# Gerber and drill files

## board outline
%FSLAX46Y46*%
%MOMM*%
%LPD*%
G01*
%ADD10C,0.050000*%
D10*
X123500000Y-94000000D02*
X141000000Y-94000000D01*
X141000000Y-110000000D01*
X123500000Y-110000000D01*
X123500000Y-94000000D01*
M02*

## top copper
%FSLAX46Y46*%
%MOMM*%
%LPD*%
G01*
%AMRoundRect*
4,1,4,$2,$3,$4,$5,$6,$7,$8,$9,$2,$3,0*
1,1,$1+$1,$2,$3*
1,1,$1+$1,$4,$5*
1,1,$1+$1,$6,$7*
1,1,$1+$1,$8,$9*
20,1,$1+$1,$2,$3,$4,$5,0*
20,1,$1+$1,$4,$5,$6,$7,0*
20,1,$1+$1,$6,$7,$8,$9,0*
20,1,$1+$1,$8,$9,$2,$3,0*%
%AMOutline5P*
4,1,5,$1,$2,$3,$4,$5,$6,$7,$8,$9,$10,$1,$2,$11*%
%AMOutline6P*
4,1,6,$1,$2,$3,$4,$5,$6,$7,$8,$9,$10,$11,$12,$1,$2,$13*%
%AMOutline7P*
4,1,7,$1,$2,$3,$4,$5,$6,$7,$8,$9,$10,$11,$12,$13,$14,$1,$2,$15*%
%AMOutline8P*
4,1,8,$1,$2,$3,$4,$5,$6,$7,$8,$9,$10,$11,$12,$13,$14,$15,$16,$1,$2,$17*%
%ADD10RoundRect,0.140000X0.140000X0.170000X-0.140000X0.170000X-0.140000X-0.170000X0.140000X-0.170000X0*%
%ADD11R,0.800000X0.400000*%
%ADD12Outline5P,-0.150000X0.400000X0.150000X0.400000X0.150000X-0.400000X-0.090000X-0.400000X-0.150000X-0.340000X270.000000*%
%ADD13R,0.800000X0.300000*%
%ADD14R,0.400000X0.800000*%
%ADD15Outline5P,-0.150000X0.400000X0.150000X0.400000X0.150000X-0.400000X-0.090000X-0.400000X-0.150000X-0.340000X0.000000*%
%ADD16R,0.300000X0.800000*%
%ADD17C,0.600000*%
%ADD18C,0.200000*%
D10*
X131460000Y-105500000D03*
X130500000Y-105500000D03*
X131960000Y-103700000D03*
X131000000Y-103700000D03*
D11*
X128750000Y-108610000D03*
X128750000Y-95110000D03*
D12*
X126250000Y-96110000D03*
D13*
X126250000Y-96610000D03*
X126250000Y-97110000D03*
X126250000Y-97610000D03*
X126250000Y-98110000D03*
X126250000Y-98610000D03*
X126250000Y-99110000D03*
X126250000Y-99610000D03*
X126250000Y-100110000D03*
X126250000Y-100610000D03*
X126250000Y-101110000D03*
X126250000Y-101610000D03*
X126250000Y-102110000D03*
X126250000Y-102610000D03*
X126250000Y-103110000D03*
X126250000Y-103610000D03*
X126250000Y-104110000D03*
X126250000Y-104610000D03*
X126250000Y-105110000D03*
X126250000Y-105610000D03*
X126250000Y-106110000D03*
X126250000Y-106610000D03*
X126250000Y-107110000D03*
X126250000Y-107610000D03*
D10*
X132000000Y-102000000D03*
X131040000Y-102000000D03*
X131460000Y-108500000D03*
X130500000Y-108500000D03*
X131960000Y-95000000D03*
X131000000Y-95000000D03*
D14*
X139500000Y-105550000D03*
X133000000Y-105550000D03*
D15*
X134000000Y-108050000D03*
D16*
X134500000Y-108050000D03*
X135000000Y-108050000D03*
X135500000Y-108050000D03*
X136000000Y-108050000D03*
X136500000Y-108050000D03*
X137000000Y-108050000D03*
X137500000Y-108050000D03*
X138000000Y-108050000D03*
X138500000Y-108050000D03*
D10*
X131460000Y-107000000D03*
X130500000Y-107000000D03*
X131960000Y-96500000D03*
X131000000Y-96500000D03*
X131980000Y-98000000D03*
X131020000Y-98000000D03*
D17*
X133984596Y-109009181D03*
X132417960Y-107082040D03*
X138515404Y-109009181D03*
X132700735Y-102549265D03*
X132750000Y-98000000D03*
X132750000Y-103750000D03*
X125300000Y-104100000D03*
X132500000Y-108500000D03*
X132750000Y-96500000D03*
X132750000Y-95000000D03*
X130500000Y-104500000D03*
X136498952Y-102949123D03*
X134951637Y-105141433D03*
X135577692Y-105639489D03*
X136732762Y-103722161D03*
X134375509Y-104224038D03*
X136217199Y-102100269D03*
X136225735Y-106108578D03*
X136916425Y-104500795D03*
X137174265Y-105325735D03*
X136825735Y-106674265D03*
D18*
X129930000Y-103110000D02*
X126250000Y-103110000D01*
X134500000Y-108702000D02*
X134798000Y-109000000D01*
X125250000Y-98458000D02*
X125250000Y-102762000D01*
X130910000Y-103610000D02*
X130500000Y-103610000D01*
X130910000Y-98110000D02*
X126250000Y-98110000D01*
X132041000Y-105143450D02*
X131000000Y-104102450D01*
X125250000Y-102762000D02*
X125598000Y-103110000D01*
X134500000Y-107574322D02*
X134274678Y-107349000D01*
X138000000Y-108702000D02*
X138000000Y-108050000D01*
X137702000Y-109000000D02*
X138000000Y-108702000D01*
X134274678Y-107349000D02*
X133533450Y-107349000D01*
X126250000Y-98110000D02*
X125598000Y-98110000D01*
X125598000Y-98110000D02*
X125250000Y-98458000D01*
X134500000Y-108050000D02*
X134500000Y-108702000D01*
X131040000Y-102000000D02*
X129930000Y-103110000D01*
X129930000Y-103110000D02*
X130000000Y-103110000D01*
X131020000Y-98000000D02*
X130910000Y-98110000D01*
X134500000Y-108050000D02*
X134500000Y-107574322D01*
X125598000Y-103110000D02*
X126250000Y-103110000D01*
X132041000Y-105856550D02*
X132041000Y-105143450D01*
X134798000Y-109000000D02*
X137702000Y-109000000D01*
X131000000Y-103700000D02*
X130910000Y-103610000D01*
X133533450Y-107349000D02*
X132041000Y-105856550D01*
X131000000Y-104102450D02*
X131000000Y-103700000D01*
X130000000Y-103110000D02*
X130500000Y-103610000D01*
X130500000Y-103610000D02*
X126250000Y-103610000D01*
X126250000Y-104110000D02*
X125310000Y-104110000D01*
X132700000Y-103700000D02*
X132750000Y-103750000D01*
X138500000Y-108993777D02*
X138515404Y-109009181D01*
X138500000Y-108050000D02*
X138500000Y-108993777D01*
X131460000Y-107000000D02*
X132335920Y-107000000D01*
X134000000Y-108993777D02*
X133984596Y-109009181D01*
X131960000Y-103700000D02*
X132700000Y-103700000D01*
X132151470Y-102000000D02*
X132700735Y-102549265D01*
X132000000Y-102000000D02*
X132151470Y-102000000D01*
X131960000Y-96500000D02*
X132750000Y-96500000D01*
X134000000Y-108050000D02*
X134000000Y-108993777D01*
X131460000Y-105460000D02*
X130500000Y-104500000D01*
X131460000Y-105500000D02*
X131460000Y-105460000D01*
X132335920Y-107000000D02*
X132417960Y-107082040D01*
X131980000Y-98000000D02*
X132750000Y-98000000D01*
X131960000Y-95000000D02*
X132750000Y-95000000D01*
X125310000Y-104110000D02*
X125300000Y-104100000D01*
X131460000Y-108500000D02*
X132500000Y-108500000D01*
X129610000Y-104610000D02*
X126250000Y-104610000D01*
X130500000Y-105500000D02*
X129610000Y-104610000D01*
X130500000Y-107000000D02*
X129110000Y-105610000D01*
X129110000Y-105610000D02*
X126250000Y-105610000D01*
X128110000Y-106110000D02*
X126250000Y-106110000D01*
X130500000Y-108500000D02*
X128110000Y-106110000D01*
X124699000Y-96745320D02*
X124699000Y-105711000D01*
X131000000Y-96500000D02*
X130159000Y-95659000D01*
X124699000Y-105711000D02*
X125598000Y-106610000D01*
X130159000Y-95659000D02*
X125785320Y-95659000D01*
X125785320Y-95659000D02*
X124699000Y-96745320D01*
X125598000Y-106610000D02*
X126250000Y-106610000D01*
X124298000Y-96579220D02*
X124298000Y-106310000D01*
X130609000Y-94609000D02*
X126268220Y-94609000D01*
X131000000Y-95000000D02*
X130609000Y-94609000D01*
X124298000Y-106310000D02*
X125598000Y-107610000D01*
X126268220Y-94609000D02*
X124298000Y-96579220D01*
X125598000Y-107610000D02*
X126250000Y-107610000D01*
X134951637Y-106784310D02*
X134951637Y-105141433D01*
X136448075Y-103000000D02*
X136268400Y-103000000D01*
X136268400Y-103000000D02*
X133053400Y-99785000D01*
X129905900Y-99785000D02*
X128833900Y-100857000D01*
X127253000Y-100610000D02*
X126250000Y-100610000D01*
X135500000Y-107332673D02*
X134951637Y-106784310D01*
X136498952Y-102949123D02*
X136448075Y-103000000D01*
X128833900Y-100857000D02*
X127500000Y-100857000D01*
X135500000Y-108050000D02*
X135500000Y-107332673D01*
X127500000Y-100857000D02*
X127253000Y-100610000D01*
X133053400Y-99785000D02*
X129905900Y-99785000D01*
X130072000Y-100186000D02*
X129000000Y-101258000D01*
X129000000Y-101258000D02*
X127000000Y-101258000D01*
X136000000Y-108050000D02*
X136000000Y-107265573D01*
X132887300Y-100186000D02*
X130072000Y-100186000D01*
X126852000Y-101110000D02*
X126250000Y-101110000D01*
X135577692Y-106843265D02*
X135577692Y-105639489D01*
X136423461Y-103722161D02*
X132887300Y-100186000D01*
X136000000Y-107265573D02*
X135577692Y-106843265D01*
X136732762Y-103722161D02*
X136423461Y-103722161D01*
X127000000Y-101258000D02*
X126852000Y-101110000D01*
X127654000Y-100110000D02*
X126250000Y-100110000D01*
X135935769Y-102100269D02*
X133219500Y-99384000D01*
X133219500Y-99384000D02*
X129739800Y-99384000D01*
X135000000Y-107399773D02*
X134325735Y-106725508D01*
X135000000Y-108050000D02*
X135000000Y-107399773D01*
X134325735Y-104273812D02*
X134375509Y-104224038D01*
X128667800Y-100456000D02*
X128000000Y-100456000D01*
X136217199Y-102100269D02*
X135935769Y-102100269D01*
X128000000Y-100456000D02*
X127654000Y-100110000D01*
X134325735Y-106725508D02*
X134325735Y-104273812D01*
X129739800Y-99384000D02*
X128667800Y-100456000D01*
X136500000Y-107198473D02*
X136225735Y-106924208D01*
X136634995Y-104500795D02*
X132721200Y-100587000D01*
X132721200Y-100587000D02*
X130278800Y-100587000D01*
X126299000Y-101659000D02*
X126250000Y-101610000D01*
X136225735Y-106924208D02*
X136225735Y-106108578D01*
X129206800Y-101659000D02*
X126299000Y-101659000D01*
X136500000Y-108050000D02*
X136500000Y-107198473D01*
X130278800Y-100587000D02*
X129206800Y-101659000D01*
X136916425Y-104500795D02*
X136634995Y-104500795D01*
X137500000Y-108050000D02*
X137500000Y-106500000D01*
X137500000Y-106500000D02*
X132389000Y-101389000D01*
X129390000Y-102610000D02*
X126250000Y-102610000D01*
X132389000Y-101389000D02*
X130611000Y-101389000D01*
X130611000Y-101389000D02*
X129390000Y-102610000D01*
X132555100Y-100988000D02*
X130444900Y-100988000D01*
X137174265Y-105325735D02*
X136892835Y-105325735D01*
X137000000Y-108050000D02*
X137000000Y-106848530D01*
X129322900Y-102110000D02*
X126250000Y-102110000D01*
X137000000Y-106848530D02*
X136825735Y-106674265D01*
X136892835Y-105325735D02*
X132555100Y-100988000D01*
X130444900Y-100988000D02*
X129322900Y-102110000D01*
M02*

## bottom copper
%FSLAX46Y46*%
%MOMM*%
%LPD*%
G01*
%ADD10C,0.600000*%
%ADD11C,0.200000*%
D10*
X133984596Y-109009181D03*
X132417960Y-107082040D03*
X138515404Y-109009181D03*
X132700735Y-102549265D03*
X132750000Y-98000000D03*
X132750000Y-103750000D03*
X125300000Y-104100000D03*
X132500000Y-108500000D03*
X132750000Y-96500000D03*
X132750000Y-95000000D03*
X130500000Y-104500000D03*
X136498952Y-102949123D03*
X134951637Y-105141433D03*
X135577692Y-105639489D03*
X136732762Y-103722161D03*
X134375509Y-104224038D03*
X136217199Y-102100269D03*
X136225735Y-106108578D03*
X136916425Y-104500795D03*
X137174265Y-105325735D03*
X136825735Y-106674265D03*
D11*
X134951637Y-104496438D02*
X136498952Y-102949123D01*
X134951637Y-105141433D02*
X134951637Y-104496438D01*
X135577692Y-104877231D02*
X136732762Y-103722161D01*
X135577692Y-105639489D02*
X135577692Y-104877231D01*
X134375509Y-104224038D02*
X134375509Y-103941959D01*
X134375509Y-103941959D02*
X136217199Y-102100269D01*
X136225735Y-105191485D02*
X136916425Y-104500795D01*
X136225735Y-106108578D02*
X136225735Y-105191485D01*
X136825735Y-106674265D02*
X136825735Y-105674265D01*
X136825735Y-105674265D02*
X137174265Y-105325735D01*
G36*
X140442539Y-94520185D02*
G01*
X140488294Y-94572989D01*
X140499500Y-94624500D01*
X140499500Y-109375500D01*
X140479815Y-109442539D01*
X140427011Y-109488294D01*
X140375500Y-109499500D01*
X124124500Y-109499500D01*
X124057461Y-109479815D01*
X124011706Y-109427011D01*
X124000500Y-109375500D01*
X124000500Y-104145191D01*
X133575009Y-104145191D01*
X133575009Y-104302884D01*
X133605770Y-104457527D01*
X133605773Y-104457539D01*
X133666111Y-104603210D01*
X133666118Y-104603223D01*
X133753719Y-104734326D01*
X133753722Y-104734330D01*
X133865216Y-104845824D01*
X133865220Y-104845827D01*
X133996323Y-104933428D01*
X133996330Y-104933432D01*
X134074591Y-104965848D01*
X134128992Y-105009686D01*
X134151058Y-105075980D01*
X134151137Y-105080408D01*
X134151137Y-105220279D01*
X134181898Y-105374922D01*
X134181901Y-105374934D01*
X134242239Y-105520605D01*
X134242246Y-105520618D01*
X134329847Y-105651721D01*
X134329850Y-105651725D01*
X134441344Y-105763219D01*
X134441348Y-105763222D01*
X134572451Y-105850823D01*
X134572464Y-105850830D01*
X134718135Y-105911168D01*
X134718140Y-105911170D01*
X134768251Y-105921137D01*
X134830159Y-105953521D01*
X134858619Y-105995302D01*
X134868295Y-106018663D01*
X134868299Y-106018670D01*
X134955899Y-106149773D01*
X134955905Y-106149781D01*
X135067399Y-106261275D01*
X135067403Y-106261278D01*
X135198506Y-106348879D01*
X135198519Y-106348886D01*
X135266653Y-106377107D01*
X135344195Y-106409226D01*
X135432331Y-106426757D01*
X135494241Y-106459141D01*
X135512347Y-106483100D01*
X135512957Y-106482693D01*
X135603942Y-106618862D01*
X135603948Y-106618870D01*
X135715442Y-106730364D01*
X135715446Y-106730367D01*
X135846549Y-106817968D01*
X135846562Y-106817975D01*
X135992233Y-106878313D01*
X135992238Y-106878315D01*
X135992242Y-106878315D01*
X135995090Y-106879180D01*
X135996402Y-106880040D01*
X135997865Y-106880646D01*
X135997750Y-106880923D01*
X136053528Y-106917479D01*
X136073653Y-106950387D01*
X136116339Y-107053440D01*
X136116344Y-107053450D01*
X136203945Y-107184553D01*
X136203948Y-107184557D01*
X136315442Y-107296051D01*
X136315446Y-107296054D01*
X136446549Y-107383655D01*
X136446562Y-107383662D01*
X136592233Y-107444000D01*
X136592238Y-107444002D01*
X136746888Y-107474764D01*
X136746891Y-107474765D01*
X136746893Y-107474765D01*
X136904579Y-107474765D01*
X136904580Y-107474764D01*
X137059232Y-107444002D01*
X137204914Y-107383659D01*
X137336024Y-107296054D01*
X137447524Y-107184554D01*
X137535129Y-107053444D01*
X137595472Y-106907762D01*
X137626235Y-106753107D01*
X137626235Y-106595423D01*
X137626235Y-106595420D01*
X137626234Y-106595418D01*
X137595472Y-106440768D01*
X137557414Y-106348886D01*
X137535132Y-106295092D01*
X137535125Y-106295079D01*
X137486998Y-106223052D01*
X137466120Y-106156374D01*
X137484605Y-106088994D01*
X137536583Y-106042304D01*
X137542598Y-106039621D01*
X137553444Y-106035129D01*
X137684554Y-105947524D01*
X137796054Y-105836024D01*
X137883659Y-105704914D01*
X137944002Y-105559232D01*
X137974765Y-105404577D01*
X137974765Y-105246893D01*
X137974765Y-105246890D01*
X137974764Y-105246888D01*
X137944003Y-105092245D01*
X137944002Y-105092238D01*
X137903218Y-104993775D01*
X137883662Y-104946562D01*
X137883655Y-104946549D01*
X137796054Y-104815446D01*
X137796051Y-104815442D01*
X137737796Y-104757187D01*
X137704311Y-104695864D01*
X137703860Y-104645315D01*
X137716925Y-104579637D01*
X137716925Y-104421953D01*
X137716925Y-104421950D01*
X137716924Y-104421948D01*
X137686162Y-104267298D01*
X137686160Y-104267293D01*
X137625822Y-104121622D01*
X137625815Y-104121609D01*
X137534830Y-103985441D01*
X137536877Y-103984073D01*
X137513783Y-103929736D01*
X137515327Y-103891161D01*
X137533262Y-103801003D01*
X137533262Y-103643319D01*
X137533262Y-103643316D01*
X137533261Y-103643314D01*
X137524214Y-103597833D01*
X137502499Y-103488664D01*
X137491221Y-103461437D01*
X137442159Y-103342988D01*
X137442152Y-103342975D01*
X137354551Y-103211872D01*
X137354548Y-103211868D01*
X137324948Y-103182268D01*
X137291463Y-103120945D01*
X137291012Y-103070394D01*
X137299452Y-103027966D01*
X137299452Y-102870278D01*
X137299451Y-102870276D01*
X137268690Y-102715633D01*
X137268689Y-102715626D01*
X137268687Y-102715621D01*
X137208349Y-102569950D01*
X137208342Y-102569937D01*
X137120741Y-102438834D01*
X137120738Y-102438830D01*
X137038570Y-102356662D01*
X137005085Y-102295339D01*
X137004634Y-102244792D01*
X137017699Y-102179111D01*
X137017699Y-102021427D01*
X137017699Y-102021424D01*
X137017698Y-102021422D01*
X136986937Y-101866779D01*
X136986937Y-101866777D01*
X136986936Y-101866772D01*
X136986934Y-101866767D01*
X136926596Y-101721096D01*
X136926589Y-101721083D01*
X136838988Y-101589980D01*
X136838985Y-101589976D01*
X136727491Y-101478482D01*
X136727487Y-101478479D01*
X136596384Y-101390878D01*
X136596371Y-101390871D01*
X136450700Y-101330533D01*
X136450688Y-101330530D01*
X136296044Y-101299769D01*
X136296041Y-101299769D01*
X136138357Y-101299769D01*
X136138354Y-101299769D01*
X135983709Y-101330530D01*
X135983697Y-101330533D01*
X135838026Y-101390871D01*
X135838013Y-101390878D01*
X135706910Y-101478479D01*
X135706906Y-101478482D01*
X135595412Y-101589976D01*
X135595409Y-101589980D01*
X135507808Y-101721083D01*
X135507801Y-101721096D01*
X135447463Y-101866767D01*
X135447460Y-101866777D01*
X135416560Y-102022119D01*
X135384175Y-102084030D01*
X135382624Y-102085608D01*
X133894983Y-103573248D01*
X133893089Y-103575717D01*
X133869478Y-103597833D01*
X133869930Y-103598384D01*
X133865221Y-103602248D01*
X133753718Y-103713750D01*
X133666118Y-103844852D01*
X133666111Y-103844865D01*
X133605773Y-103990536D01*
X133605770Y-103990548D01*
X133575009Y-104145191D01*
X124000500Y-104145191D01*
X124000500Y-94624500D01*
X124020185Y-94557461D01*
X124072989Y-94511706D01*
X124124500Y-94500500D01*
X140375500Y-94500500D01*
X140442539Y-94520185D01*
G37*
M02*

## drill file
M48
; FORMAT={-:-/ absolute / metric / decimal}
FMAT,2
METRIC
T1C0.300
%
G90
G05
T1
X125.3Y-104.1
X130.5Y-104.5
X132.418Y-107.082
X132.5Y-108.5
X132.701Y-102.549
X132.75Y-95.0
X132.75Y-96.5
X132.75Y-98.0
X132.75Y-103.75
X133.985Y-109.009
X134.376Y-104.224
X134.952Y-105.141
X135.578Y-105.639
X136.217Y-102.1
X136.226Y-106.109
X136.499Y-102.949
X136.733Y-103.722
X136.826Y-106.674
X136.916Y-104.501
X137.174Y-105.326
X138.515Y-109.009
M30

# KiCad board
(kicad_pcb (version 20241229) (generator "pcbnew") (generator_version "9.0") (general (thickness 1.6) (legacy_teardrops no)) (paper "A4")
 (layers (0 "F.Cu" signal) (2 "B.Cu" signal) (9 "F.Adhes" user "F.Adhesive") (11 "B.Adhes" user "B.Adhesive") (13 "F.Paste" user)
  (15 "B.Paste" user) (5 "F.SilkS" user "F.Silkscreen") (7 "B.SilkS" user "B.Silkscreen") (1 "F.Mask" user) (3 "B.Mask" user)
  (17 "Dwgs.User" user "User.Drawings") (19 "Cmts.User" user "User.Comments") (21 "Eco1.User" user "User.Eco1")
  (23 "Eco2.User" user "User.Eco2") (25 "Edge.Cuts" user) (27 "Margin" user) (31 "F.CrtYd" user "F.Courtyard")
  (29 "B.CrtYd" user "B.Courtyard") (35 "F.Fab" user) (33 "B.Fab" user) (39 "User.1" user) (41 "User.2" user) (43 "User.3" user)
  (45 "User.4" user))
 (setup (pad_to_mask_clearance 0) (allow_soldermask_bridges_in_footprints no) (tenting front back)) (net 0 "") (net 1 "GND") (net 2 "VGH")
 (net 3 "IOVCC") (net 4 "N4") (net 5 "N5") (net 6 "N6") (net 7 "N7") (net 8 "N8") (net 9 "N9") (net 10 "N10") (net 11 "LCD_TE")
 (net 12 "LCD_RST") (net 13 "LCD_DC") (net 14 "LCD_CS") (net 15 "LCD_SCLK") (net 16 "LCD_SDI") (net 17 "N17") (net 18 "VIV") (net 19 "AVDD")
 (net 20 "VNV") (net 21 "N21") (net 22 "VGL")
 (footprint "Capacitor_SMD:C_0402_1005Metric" (layer "F.Cu") (at 130.98 105.5 180)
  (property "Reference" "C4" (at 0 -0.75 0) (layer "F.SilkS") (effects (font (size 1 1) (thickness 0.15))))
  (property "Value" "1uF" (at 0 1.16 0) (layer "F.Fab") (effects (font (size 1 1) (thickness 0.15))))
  (pad "1" smd roundrect (at -0.48 0 180) (size 0.56 0.62) (layers "F.Cu" "F.Mask" "F.Paste") (roundrect_rratio 0.25) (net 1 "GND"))
  (pad "2" smd roundrect (at 0.48 0 180) (size 0.56 0.62) (layers "F.Cu" "F.Mask" "F.Paste") (roundrect_rratio 0.25) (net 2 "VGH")))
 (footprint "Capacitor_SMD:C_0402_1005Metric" (layer "F.Cu") (at 131.48 103.7 180)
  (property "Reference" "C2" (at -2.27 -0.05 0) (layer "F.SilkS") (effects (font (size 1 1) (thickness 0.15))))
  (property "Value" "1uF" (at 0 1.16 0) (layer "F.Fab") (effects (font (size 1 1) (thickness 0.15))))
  (pad "1" smd roundrect (at -0.48 0 180) (size 0.56 0.62) (layers "F.Cu" "F.Mask" "F.Paste") (roundrect_rratio 0.25) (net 1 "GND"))
  (pad "2" smd roundrect (at 0.48 0 180) (size 0.56 0.62) (layers "F.Cu" "F.Mask" "F.Paste") (roundrect_rratio 0.25) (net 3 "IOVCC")))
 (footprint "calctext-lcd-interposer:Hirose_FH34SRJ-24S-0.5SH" (layer "F.Cu") (at 126.25 101.86 90)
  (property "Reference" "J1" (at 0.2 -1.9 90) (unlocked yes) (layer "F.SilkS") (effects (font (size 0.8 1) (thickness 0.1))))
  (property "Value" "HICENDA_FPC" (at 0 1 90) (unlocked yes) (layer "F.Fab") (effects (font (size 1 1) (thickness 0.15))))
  (pad "" smd rect (at -6.75 2.5 90) (size 0.4 0.8) (layers "F.Cu" "F.Mask" "F.Paste") (thermal_bridge_angle 45))
  (pad "" smd rect (at 6.75 2.5 90) (size 0.4 0.8) (layers "F.Cu" "F.Mask" "F.Paste") (thermal_bridge_angle 45))
  (pad "1" smd roundrect (at 5.75 0 270) (size 0.3 0.8) (layers "F.Cu" "F.Mask" "F.Paste") (roundrect_rratio 0) (chamfer_ratio 0.2)
   (chamfer bottom_left) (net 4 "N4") (thermal_bridge_angle 45))
  (pad "2" smd rect (at 5.25 0 270) (size 0.3 0.8) (layers "F.Cu" "F.Mask" "F.Paste") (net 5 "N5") (thermal_bridge_angle 45))
  (pad "3" smd rect (at 4.75 0 270) (size 0.3 0.8) (layers "F.Cu" "F.Mask" "F.Paste") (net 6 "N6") (thermal_bridge_angle 45))
  (pad "4" smd rect (at 4.25 0 270) (size 0.3 0.8) (layers "F.Cu" "F.Mask" "F.Paste") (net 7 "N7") (thermal_bridge_angle 45))
  (pad "5" smd rect (at 3.75 0 270) (size 0.3 0.8) (layers "F.Cu" "F.Mask" "F.Paste") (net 3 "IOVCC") (thermal_bridge_angle 45))
  (pad "6" smd rect (at 3.25 0 270) (size 0.3 0.8) (layers "F.Cu" "F.Mask" "F.Paste") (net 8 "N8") (thermal_bridge_angle 45))
  (pad "7" smd rect (at 2.75 0 270) (size 0.3 0.8) (layers "F.Cu" "F.Mask" "F.Paste") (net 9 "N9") (thermal_bridge_angle 45))
  (pad "8" smd rect (at 2.25 0 270) (size 0.3 0.8) (layers "F.Cu" "F.Mask" "F.Paste") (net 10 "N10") (thermal_bridge_angle 45))
  (pad "9" smd rect (at 1.75 0 270) (size 0.3 0.8) (layers "F.Cu" "F.Mask" "F.Paste") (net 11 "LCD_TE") (thermal_bridge_angle 45))
  (pad "10" smd rect (at 1.25 0 270) (size 0.3 0.8) (layers "F.Cu" "F.Mask" "F.Paste") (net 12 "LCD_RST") (thermal_bridge_angle 45))
  (pad "11" smd rect (at 0.75 0 270) (size 0.3 0.8) (layers "F.Cu" "F.Mask" "F.Paste") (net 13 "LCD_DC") (thermal_bridge_angle 45))
  (pad "12" smd rect (at 0.25 0 270) (size 0.3 0.8) (layers "F.Cu" "F.Mask" "F.Paste") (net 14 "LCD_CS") (thermal_bridge_angle 45))
  (pad "13" smd rect (at -0.25 0 270) (size 0.3 0.8) (layers "F.Cu" "F.Mask" "F.Paste") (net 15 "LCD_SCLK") (thermal_bridge_angle 45))
  (pad "14" smd rect (at -0.75 0 270) (size 0.3 0.8) (layers "F.Cu" "F.Mask" "F.Paste") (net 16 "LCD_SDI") (thermal_bridge_angle 45))
  (pad "15" smd rect (at -1.25 0 270) (size 0.3 0.8) (layers "F.Cu" "F.Mask" "F.Paste") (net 3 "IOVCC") (thermal_bridge_angle 45))
  (pad "16" smd rect (at -1.75 0 270) (size 0.3 0.8) (layers "F.Cu" "F.Mask" "F.Paste") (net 3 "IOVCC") (thermal_bridge_angle 45))
  (pad "17" smd rect (at -2.25 0 270) (size 0.3 0.8) (layers "F.Cu" "F.Mask" "F.Paste") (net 1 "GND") (thermal_bridge_angle 45))
  (pad "18" smd rect (at -2.75 0 270) (size 0.3 0.8) (layers "F.Cu" "F.Mask" "F.Paste") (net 2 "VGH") (thermal_bridge_angle 45))
  (pad "19" smd rect (at -3.25 0 270) (size 0.3 0.8) (layers "F.Cu" "F.Mask" "F.Paste") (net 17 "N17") (thermal_bridge_angle 45))
  (pad "20" smd rect (at -3.75 0 270) (size 0.3 0.8) (layers "F.Cu" "F.Mask" "F.Paste") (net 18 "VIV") (thermal_bridge_angle 45))
  (pad "21" smd rect (at -4.25 0 270) (size 0.3 0.8) (layers "F.Cu" "F.Mask" "F.Paste") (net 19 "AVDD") (thermal_bridge_angle 45))
  (pad "22" smd rect (at -4.75 0 270) (size 0.3 0.8) (layers "F.Cu" "F.Mask" "F.Paste") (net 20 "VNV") (thermal_bridge_angle 45))
  (pad "23" smd rect (at -5.25 0 270) (size 0.3 0.8) (layers "F.Cu" "F.Mask" "F.Paste") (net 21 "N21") (thermal_bridge_angle 45))
  (pad "24" smd rect (at -5.75 0 270) (size 0.3 0.8) (layers "F.Cu" "F.Mask" "F.Paste") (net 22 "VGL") (thermal_bridge_angle 45)))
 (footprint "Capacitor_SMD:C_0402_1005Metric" (layer "F.Cu") (at 131.52 102 180)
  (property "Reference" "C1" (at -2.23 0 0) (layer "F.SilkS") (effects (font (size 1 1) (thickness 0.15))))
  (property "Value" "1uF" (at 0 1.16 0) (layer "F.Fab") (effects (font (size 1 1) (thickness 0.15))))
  (pad "1" smd roundrect (at -0.48 0 180) (size 0.56 0.62) (layers "F.Cu" "F.Mask" "F.Paste") (roundrect_rratio 0.25) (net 1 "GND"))
  (pad "2" smd roundrect (at 0.48 0 180) (size 0.56 0.62) (layers "F.Cu" "F.Mask" "F.Paste") (roundrect_rratio 0.25) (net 3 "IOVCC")))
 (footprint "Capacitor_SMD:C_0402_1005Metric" (layer "F.Cu") (at 130.98 108.5 180)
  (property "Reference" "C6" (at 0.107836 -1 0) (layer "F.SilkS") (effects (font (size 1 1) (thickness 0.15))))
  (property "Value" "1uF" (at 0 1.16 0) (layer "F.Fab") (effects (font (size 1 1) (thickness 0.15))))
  (pad "1" smd roundrect (at -0.48 0 180) (size 0.56 0.62) (layers "F.Cu" "F.Mask" "F.Paste") (roundrect_rratio 0.25) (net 1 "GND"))
  (pad "2" smd roundrect (at 0.48 0 180) (size 0.56 0.62) (layers "F.Cu" "F.Mask" "F.Paste") (roundrect_rratio 0.25) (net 19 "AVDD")))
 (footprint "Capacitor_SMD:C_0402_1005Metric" (layer "F.Cu") (at 131.48 95 180)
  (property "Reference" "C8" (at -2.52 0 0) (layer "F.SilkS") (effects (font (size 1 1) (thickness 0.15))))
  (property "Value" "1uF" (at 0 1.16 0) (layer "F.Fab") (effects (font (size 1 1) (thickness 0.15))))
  (pad "1" smd roundrect (at -0.48 0 180) (size 0.56 0.62) (layers "F.Cu" "F.Mask" "F.Paste") (roundrect_rratio 0.25) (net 1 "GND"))
  (pad "2" smd roundrect (at 0.48 0 180) (size 0.56 0.62) (layers "F.Cu" "F.Mask" "F.Paste") (roundrect_rratio 0.25) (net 22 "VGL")))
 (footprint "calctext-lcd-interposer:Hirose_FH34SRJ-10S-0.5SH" (layer "F.Cu") (at 136.25 108.05 180)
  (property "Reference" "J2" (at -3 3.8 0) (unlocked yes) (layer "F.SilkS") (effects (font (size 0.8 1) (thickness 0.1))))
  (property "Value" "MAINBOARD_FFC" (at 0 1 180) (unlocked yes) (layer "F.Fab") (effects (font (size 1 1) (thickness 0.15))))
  (pad "" smd rect (at -3.25 2.5 180) (size 0.4 0.8) (layers "F.Cu" "F.Mask" "F.Paste") (thermal_bridge_angle 45))
  (pad "" smd rect (at 3.25 2.5 180) (size 0.4 0.8) (layers "F.Cu" "F.Mask" "F.Paste") (thermal_bridge_angle 45))
  (pad "1" smd roundrect (at 2.25 0) (size 0.3 0.8) (layers "F.Cu" "F.Mask" "F.Paste") (roundrect_rratio 0) (chamfer_ratio 0.2)
   (chamfer bottom_left) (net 1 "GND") (thermal_bridge_angle 45))
  (pad "2" smd rect (at 1.75 0) (size 0.3 0.8) (layers "F.Cu" "F.Mask" "F.Paste") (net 3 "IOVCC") (thermal_bridge_angle 45))
  (pad "3" smd rect (at 1.25 0) (size 0.3 0.8) (layers "F.Cu" "F.Mask" "F.Paste") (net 11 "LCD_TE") (thermal_bridge_angle 45))
  (pad "4" smd rect (at 0.75 0) (size 0.3 0.8) (layers "F.Cu" "F.Mask" "F.Paste") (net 12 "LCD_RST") (thermal_bridge_angle 45))
  (pad "5" smd rect (at 0.25 0) (size 0.3 0.8) (layers "F.Cu" "F.Mask" "F.Paste") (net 13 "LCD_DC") (thermal_bridge_angle 45))
  (pad "6" smd rect (at -0.25 0) (size 0.3 0.8) (layers "F.Cu" "F.Mask" "F.Paste") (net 14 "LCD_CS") (thermal_bridge_angle 45))
  (pad "7" smd rect (at -0.75 0) (size 0.3 0.8) (layers "F.Cu" "F.Mask" "F.Paste") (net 15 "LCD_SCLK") (thermal_bridge_angle 45))
  (pad "8" smd rect (at -1.25 0) (size 0.3 0.8) (layers "F.Cu" "F.Mask" "F.Paste") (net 16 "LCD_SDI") (thermal_bridge_angle 45))
  (pad "9" smd rect (at -1.75 0) (size 0.3 0.8) (layers "F.Cu" "F.Mask" "F.Paste") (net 3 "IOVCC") (thermal_bridge_angle 45))
  (pad "10" smd rect (at -2.25 0) (size 0.3 0.8) (layers "F.Cu" "F.Mask" "F.Paste") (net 1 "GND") (thermal_bridge_angle 45)))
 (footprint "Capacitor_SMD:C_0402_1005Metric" (layer "F.Cu") (at 130.98 107 180)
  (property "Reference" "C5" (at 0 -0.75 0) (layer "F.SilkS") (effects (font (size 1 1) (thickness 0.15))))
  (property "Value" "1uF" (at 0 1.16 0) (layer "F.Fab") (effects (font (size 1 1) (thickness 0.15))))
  (pad "1" smd roundrect (at -0.48 0 180) (size 0.56 0.62) (layers "F.Cu" "F.Mask" "F.Paste") (roundrect_rratio 0.25) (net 1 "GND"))
  (pad "2" smd roundrect (at 0.48 0 180) (size 0.56 0.62) (layers "F.Cu" "F.Mask" "F.Paste") (roundrect_rratio 0.25) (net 18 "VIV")))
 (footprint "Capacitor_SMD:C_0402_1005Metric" (layer "F.Cu") (at 131.48 96.5 180)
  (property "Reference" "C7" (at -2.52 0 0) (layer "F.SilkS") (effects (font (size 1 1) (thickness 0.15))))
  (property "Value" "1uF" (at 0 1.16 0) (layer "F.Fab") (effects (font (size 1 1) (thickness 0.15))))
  (pad "1" smd roundrect (at -0.48 0 180) (size 0.56 0.62) (layers "F.Cu" "F.Mask" "F.Paste") (roundrect_rratio 0.25) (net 1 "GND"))
  (pad "2" smd roundrect (at 0.48 0 180) (size 0.56 0.62) (layers "F.Cu" "F.Mask" "F.Paste") (roundrect_rratio 0.25) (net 20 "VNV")))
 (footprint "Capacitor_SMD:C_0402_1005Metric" (layer "F.Cu") (at 131.5 98 180)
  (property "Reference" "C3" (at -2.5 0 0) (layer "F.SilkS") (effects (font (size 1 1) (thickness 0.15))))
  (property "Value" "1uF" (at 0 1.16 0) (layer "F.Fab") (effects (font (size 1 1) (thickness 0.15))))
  (pad "1" smd roundrect (at -0.48 0 180) (size 0.56 0.62) (layers "F.Cu" "F.Mask" "F.Paste") (roundrect_rratio 0.25) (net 1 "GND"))
  (pad "2" smd roundrect (at 0.48 0 180) (size 0.56 0.62) (layers "F.Cu" "F.Mask" "F.Paste") (roundrect_rratio 0.25) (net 3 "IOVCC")))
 (gr_rect (start 123.5 94) (end 141 110) (stroke (width 0.05) (type default)) (fill no) (layer "Edge.Cuts"))
 (segment (start 129.93 103.11) (end 126.25 103.11) (width 0.2) (layer "F.Cu") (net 3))
 (segment (start 134.5 108.702) (end 134.798 109) (width 0.2) (layer "F.Cu") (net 3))
 (segment (start 125.25 98.458) (end 125.25 102.762) (width 0.2) (layer "F.Cu") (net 3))
 (segment (start 130.91 103.61) (end 130.5 103.61) (width 0.2) (layer "F.Cu") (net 3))
 (segment (start 130.91 98.11) (end 126.25 98.11) (width 0.2) (layer "F.Cu") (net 3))
 (segment (start 132.041 105.14345) (end 131 104.10245) (width 0.2) (layer "F.Cu") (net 3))
 (segment (start 125.25 102.762) (end 125.598 103.11) (width 0.2) (layer "F.Cu") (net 3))
 (segment (start 134.5 107.574322) (end 134.274678 107.349) (width 0.2) (layer "F.Cu") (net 3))
 (segment (start 138 108.702) (end 138 108.05) (width 0.2) (layer "F.Cu") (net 3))
 (segment (start 137.702 109) (end 138 108.702) (width 0.2) (layer "F.Cu") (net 3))
 (segment (start 134.274678 107.349) (end 133.53345 107.349) (width 0.2) (layer "F.Cu") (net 3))
 (segment (start 126.25 98.11) (end 125.598 98.11) (width 0.2) (layer "F.Cu") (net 3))
 (segment (start 125.598 98.11) (end 125.25 98.458) (width 0.2) (layer "F.Cu") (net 3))
 (segment (start 134.5 108.05) (end 134.5 108.702) (width 0.2) (layer "F.Cu") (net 3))
 (segment (start 131.04 102) (end 129.93 103.11) (width 0.2) (layer "F.Cu") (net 3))
 (segment (start 129.93 103.11) (end 130 103.11) (width 0.2) (layer "F.Cu") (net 3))
 (segment (start 131.02 98) (end 130.91 98.11) (width 0.2) (layer "F.Cu") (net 3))
 (segment (start 134.5 108.05) (end 134.5 107.574322) (width 0.2) (layer "F.Cu") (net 3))
 (segment (start 125.598 103.11) (end 126.25 103.11) (width 0.2) (layer "F.Cu") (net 3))
 (segment (start 132.041 105.85655) (end 132.041 105.14345) (width 0.2) (layer "F.Cu") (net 3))
 (segment (start 134.798 109) (end 137.702 109) (width 0.2) (layer "F.Cu") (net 3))
 (segment (start 131 103.7) (end 130.91 103.61) (width 0.2) (layer "F.Cu") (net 3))
 (segment (start 133.53345 107.349) (end 132.041 105.85655) (width 0.2) (layer "F.Cu") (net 3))
 (segment (start 131 104.10245) (end 131 103.7) (width 0.2) (layer "F.Cu") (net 3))
 (segment (start 130 103.11) (end 130.5 103.61) (width 0.2) (layer "F.Cu") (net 3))
 (segment (start 130.5 103.61) (end 126.25 103.61) (width 0.2) (layer "F.Cu") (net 3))
 (segment (start 126.25 104.11) (end 125.31 104.11) (width 0.2) (layer "F.Cu") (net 1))
 (segment (start 132.7 103.7) (end 132.75 103.75) (width 0.2) (layer "F.Cu") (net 1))
 (segment (start 138.5 108.993777) (end 138.515404 109.009181) (width 0.2) (layer "F.Cu") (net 1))
 (segment (start 138.5 108.05) (end 138.5 108.993777) (width 0.2) (layer "F.Cu") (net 1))
 (segment (start 131.46 107) (end 132.33592 107) (width 0.2) (layer "F.Cu") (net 1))
 (segment (start 134 108.993777) (end 133.984596 109.009181) (width 0.2) (layer "F.Cu") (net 1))
 (segment (start 131.96 103.7) (end 132.7 103.7) (width 0.2) (layer "F.Cu") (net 1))
 (segment (start 132.15147 102) (end 132.700735 102.549265) (width 0.2) (layer "F.Cu") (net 1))
 (segment (start 132 102) (end 132.15147 102) (width 0.2) (layer "F.Cu") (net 1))
 (segment (start 131.96 96.5) (end 132.75 96.5) (width 0.2) (layer "F.Cu") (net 1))
 (segment (start 134 108.05) (end 134 108.993777) (width 0.2) (layer "F.Cu") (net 1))
 (segment (start 131.46 105.46) (end 130.5 104.5) (width 0.2) (layer "F.Cu") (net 1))
 (segment (start 131.46 105.5) (end 131.46 105.46) (width 0.2) (layer "F.Cu") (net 1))
 (segment (start 132.33592 107) (end 132.41796 107.08204) (width 0.2) (layer "F.Cu") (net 1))
 (segment (start 131.98 98) (end 132.75 98) (width 0.2) (layer "F.Cu") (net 1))
 (segment (start 131.96 95) (end 132.75 95) (width 0.2) (layer "F.Cu") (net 1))
 (segment (start 125.31 104.11) (end 125.3 104.1) (width 0.2) (layer "F.Cu") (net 1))
 (segment (start 131.46 108.5) (end 132.5 108.5) (width 0.2) (layer "F.Cu") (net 1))
 (via (at 133.984596 109.009181) (size 0.6) (drill 0.3) (layers "F.Cu" "B.Cu") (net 1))
 (via (at 132.41796 107.08204) (size 0.6) (drill 0.3) (layers "F.Cu" "B.Cu") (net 1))
 (via (at 138.515404 109.009181) (size 0.6) (drill 0.3) (layers "F.Cu" "B.Cu") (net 1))
 (via (at 132.700735 102.549265) (size 0.6) (drill 0.3) (layers "F.Cu" "B.Cu") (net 1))
 (via (at 132.75 98) (size 0.6) (drill 0.3) (layers "F.Cu" "B.Cu") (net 1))
 (via (at 132.75 103.75) (size 0.6) (drill 0.3) (layers "F.Cu" "B.Cu") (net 1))
 (via (at 125.3 104.1) (size 0.6) (drill 0.3) (layers "F.Cu" "B.Cu") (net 1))
 (via (at 132.5 108.5) (size 0.6) (drill 0.3) (layers "F.Cu" "B.Cu") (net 1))
 (via (at 132.75 96.5) (size 0.6) (drill 0.3) (layers "F.Cu" "B.Cu") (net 1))
 (via (at 132.75 95) (size 0.6) (drill 0.3) (layers "F.Cu" "B.Cu") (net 1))
 (via (at 130.5 104.5) (size 0.6) (drill 0.3) (layers "F.Cu" "B.Cu") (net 1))
 (segment (start 129.61 104.61) (end 126.25 104.61) (width 0.2) (layer "F.Cu") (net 2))
 (segment (start 130.5 105.5) (end 129.61 104.61) (width 0.2) (layer "F.Cu") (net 2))
 (segment (start 130.5 107) (end 129.11 105.61) (width 0.2) (layer "F.Cu") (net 18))
 (segment (start 129.11 105.61) (end 126.25 105.61) (width 0.2) (layer "F.Cu") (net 18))
 (segment (start 128.11 106.11) (end 126.25 106.11) (width 0.2) (layer "F.Cu") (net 19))
 (segment (start 130.5 108.5) (end 128.11 106.11) (width 0.2) (layer "F.Cu") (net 19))
 (segment (start 124.699 96.74532) (end 124.699 105.711) (width 0.2) (layer "F.Cu") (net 20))
 (segment (start 131 96.5) (end 130.159 95.659) (width 0.2) (layer "F.Cu") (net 20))
 (segment (start 124.699 105.711) (end 125.598 106.61) (width 0.2) (layer "F.Cu") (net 20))
 (segment (start 130.159 95.659) (end 125.78532 95.659) (width 0.2) (layer "F.Cu") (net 20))
 (segment (start 125.78532 95.659) (end 124.699 96.74532) (width 0.2) (layer "F.Cu") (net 20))
 (segment (start 125.598 106.61) (end 126.25 106.61) (width 0.2) (layer "F.Cu") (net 20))
 (segment (start 124.298 96.57922) (end 124.298 106.31) (width 0.2) (layer "F.Cu") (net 22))
 (segment (start 130.609 94.609) (end 126.26822 94.609) (width 0.2) (layer "F.Cu") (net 22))
 (segment (start 131 95) (end 130.609 94.609) (width 0.2) (layer "F.Cu") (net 22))
 (segment (start 124.298 106.31) (end 125.598 107.61) (width 0.2) (layer "F.Cu") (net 22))
 (segment (start 126.26822 94.609) (end 124.298 96.57922) (width 0.2) (layer "F.Cu") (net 22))
 (segment (start 125.598 107.61) (end 126.25 107.61) (width 0.2) (layer "F.Cu") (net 22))
 (segment (start 134.951637 106.78431) (end 134.951637 105.141433) (width 0.2) (layer "F.Cu") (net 12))
 (segment (start 136.448075 103) (end 136.2684 103) (width 0.2) (layer "F.Cu") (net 12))
 (segment (start 136.2684 103) (end 133.0534 99.785) (width 0.2) (layer "F.Cu") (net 12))
 (segment (start 129.9059 99.785) (end 128.8339 100.857) (width 0.2) (layer "F.Cu") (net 12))
 (segment (start 127.253 100.61) (end 126.25 100.61) (width 0.2) (layer "F.Cu") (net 12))
 (segment (start 135.5 107.332673) (end 134.951637 106.78431) (width 0.2) (layer "F.Cu") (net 12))
 (segment (start 136.498952 102.949123) (end 136.448075 103) (width 0.2) (layer "F.Cu") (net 12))
 (segment (start 128.8339 100.857) (end 127.5 100.857) (width 0.2) (layer "F.Cu") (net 12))
 (segment (start 135.5 108.05) (end 135.5 107.332673) (width 0.2) (layer "F.Cu") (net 12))
 (segment (start 127.5 100.857) (end 127.253 100.61) (width 0.2) (layer "F.Cu") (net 12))
 (segment (start 133.0534 99.785) (end 129.9059 99.785) (width 0.2) (layer "F.Cu") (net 12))
 (via (at 136.498952 102.949123) (size 0.6) (drill 0.3) (layers "F.Cu" "B.Cu") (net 12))
 (via (at 134.951637 105.141433) (size 0.6) (drill 0.3) (layers "F.Cu" "B.Cu") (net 12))
 (segment (start 134.951637 104.496438) (end 136.498952 102.949123) (width 0.2) (layer "B.Cu") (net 12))
 (segment (start 134.951637 105.141433) (end 134.951637 104.496438) (width 0.2) (layer "B.Cu") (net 12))
 (segment (start 130.072 100.186) (end 129 101.258) (width 0.2) (layer "F.Cu") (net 13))
 (segment (start 129 101.258) (end 127 101.258) (width 0.2) (layer "F.Cu") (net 13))
 (segment (start 136 108.05) (end 136 107.265573) (width 0.2) (layer "F.Cu") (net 13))
 (segment (start 132.8873 100.186) (end 130.072 100.186) (width 0.2) (layer "F.Cu") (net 13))
 (segment (start 126.852 101.11) (end 126.25 101.11) (width 0.2) (layer "F.Cu") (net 13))
 (segment (start 135.577692 106.843265) (end 135.577692 105.639489) (width 0.2) (layer "F.Cu") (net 13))
 (segment (start 136.423461 103.722161) (end 132.8873 100.186) (width 0.2) (layer "F.Cu") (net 13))
 (segment (start 136 107.265573) (end 135.577692 106.843265) (width 0.2) (layer "F.Cu") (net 13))
 (segment (start 136.732762 103.722161) (end 136.423461 103.722161) (width 0.2) (layer "F.Cu") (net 13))
 (segment (start 127 101.258) (end 126.852 101.11) (width 0.2) (layer "F.Cu") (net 13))
 (via (at 135.577692 105.639489) (size 0.6) (drill 0.3) (layers "F.Cu" "B.Cu") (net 13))
 (via (at 136.732762 103.722161) (size 0.6) (drill 0.3) (layers "F.Cu" "B.Cu") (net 13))
 (segment (start 135.577692 104.877231) (end 136.732762 103.722161) (width 0.2) (layer "B.Cu") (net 13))
 (segment (start 135.577692 105.639489) (end 135.577692 104.877231) (width 0.2) (layer "B.Cu") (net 13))
 (segment (start 127.654 100.11) (end 126.25 100.11) (width 0.2) (layer "F.Cu") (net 11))
 (segment (start 135.935769 102.100269) (end 133.2195 99.384) (width 0.2) (layer "F.Cu") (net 11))
 (segment (start 133.2195 99.384) (end 129.7398 99.384) (width 0.2) (layer "F.Cu") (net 11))
 (segment (start 135 107.399773) (end 134.325735 106.725508) (width 0.2) (layer "F.Cu") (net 11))
 (segment (start 135 108.05) (end 135 107.399773) (width 0.2) (layer "F.Cu") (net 11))
 (segment (start 134.325735 104.273812) (end 134.375509 104.224038) (width 0.2) (layer "F.Cu") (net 11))
 (segment (start 128.6678 100.456) (end 128 100.456) (width 0.2) (layer "F.Cu") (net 11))
 (segment (start 136.217199 102.100269) (end 135.935769 102.100269) (width 0.2) (layer "F.Cu") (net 11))
 (segment (start 128 100.456) (end 127.654 100.11) (width 0.2) (layer "F.Cu") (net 11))
 (segment (start 134.325735 106.725508) (end 134.325735 104.273812) (width 0.2) (layer "F.Cu") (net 11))
 (segment (start 129.7398 99.384) (end 128.6678 100.456) (width 0.2) (layer "F.Cu") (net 11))
 (via (at 134.375509 104.224038) (size 0.6) (drill 0.3) (layers "F.Cu" "B.Cu") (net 11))
 (via (at 136.217199 102.100269) (size 0.6) (drill 0.3) (layers "F.Cu" "B.Cu") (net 11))
 (segment (start 134.375509 104.224038) (end 134.375509 103.941959) (width 0.2) (layer "B.Cu") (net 11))
 (segment (start 134.375509 103.941959) (end 136.217199 102.100269) (width 0.2) (layer "B.Cu") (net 11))
 (segment (start 136.5 107.198473) (end 136.225735 106.924208) (width 0.2) (layer "F.Cu") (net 14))
 (segment (start 136.634995 104.500795) (end 132.7212 100.587) (width 0.2) (layer "F.Cu") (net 14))
 (segment (start 132.7212 100.587) (end 130.2788 100.587) (width 0.2) (layer "F.Cu") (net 14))
 (segment (start 126.299 101.659) (end 126.25 101.61) (width 0.2) (layer "F.Cu") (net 14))
 (segment (start 136.225735 106.924208) (end 136.225735 106.108578) (width 0.2) (layer "F.Cu") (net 14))
 (segment (start 129.2068 101.659) (end 126.299 101.659) (width 0.2) (layer "F.Cu") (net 14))
 (segment (start 136.5 108.05) (end 136.5 107.198473) (width 0.2) (layer "F.Cu") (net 14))
 (segment (start 130.2788 100.587) (end 129.2068 101.659) (width 0.2) (layer "F.Cu") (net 14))
 (segment (start 136.916425 104.500795) (end 136.634995 104.500795) (width 0.2) (layer "F.Cu") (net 14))
 (via (at 136.225735 106.108578) (size 0.6) (drill 0.3) (layers "F.Cu" "B.Cu") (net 14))
 (via (at 136.916425 104.500795) (size 0.6) (drill 0.3) (layers "F.Cu" "B.Cu") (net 14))
 (segment (start 136.225735 105.191485) (end 136.916425 104.500795) (width 0.2) (layer "B.Cu") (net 14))
 (segment (start 136.225735 106.108578) (end 136.225735 105.191485) (width 0.2) (layer "B.Cu") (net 14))
 (segment (start 137.5 108.05) (end 137.5 106.5) (width 0.2) (layer "F.Cu") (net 16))
 (segment (start 137.5 106.5) (end 132.389 101.389) (width 0.2) (layer "F.Cu") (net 16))
 (segment (start 129.39 102.61) (end 126.25 102.61) (width 0.2) (layer "F.Cu") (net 16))
 (segment (start 132.389 101.389) (end 130.611 101.389) (width 0.2) (layer "F.Cu") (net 16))
 (segment (start 130.611 101.389) (end 129.39 102.61) (width 0.2) (layer "F.Cu") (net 16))
 (segment (start 132.5551 100.988) (end 130.4449 100.988) (width 0.2) (layer "F.Cu") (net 15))
 (segment (start 137.174265 105.325735) (end 136.892835 105.325735) (width 0.2) (layer "F.Cu") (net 15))
 (segment (start 137 108.05) (end 137 106.84853) (width 0.2) (layer "F.Cu") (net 15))
 (segment (start 129.3229 102.11) (end 126.25 102.11) (width 0.2) (layer "F.Cu") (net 15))
 (segment (start 137 106.84853) (end 136.825735 106.674265) (width 0.2) (layer "F.Cu") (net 15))
 (segment (start 136.892835 105.325735) (end 132.5551 100.988) (width 0.2) (layer "F.Cu") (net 15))
 (segment (start 130.4449 100.988) (end 129.3229 102.11) (width 0.2) (layer "F.Cu") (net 15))
 (via (at 137.174265 105.325735) (size 0.6) (drill 0.3) (layers "F.Cu" "B.Cu") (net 15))
 (via (at 136.825735 106.674265) (size 0.6) (drill 0.3) (layers "F.Cu" "B.Cu") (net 15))
 (segment (start 136.825735 106.674265) (end 136.825735 105.674265) (width 0.2) (layer "B.Cu") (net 15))
 (segment (start 136.825735 105.674265) (end 137.174265 105.325735) (width 0.2) (layer "B.Cu") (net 15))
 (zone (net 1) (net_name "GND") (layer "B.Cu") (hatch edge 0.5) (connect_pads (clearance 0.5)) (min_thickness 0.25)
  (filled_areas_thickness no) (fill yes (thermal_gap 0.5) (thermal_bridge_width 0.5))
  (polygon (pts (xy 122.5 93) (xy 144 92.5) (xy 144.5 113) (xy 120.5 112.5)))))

